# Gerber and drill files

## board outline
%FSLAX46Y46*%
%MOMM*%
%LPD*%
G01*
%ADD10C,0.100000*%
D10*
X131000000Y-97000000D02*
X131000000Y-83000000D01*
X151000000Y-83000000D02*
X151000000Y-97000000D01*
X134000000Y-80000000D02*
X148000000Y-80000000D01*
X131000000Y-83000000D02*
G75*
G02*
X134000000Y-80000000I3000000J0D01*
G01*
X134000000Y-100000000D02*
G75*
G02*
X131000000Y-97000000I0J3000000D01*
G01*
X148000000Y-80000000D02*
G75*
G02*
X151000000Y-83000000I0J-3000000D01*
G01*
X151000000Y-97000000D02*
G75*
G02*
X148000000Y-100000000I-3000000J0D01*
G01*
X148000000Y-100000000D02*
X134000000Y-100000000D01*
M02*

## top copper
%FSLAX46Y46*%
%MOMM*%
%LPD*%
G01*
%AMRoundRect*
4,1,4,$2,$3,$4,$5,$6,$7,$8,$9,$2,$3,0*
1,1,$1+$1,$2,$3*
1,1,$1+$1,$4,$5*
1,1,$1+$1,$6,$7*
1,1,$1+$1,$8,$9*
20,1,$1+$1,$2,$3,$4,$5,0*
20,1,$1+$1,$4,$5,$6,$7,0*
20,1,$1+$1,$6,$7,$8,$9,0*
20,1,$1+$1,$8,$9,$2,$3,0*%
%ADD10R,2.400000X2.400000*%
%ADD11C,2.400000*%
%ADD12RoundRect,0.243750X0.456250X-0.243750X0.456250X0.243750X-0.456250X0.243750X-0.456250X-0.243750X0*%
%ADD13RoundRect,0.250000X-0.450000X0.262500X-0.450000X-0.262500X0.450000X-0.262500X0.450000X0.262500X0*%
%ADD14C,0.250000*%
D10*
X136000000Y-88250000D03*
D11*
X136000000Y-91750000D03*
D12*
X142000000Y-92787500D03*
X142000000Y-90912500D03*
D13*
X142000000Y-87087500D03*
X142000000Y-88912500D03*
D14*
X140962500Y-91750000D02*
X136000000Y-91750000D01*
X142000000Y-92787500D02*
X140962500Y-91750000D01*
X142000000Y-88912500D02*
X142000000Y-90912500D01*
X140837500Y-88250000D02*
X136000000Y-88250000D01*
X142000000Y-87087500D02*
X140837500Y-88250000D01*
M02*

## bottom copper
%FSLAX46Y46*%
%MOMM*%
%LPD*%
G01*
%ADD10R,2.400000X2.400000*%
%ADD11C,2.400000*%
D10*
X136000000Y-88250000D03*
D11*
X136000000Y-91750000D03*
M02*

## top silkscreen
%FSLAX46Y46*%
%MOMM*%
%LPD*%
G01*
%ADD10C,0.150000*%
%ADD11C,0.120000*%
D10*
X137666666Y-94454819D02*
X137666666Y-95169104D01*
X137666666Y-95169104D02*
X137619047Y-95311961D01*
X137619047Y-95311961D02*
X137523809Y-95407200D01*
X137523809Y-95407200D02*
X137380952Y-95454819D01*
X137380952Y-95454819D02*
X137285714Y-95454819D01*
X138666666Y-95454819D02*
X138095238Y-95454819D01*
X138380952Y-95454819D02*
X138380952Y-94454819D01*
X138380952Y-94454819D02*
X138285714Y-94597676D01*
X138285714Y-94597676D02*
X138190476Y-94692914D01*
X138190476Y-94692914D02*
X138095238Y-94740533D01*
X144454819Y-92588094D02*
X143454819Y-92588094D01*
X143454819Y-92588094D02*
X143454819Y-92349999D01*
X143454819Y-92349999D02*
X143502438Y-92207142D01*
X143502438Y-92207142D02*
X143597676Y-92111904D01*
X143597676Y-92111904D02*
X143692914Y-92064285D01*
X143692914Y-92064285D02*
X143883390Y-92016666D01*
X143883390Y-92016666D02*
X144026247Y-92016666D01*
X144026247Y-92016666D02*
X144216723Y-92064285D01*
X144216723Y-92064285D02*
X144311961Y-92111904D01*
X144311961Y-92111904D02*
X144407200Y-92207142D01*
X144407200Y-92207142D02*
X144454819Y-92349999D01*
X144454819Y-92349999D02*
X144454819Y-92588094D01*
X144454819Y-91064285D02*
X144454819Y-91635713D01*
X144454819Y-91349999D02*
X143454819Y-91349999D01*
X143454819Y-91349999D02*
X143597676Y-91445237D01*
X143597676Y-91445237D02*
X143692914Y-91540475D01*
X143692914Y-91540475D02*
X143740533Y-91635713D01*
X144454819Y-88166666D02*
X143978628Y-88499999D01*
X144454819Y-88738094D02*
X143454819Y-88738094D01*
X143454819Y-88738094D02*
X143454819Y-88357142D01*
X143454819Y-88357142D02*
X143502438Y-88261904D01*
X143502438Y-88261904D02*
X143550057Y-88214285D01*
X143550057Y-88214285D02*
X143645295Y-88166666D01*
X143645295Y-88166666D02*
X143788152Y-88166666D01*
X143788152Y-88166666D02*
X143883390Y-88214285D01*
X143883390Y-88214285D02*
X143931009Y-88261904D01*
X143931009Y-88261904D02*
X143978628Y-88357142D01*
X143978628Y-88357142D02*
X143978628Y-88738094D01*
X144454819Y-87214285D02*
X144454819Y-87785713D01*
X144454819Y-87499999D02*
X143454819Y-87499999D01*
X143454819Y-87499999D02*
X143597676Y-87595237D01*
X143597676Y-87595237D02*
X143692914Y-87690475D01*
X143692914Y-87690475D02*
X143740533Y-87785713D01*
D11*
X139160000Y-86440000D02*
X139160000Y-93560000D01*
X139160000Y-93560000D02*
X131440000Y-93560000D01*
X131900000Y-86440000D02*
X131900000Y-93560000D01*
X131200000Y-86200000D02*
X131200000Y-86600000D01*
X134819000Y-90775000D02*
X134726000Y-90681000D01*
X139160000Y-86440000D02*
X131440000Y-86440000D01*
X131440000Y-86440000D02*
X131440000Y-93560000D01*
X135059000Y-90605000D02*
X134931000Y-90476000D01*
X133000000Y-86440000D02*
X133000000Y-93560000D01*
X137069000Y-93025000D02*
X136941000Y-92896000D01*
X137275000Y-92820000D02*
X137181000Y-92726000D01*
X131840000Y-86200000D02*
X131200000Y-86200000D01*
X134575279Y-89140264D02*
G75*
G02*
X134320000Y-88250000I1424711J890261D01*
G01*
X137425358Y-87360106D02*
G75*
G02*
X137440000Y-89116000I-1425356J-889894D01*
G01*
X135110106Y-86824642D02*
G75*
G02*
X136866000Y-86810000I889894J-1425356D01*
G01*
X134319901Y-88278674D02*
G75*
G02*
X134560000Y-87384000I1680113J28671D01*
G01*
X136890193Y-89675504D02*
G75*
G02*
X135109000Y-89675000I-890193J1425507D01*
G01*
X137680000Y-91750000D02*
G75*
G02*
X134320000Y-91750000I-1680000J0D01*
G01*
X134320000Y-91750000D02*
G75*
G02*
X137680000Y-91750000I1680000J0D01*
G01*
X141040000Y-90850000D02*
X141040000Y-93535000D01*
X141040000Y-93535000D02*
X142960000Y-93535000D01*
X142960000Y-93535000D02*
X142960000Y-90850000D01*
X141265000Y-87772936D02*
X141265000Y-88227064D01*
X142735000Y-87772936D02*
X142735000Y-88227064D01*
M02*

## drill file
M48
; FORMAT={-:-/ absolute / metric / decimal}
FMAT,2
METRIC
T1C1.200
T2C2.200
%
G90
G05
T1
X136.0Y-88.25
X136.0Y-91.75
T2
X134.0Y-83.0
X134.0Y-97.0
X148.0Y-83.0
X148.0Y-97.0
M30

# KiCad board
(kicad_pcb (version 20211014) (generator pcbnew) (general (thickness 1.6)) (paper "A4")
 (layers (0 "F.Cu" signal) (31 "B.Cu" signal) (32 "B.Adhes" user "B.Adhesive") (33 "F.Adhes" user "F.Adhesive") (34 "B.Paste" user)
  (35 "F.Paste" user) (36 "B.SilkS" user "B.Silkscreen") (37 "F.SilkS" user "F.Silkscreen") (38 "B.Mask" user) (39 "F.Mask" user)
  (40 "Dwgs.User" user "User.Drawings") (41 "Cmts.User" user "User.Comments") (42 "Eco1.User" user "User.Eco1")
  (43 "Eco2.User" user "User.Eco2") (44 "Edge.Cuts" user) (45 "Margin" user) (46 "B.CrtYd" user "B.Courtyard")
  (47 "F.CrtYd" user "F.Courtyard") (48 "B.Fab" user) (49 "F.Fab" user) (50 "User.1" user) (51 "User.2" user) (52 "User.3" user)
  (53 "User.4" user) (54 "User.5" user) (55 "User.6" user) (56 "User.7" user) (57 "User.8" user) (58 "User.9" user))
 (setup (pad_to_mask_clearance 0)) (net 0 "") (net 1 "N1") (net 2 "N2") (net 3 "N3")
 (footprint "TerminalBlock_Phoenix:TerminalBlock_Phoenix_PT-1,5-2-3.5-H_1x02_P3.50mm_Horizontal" (layer "F.Cu") (at 136 88.25 -90)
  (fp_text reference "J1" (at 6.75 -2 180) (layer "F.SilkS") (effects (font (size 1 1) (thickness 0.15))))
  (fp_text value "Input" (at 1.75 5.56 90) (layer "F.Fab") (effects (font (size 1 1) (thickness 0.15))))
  (fp_line (start -1.81 -3.16) (end 5.31 -3.16) (layer "F.SilkS") (width 0.12))
  (fp_line (start 5.31 -3.16) (end 5.31 4.56) (layer "F.SilkS") (width 0.12))
  (fp_line (start -1.81 4.1) (end 5.31 4.1) (layer "F.SilkS") (width 0.12))
  (fp_line (start -2.05 4.8) (end -1.65 4.8) (layer "F.SilkS") (width 0.12))
  (fp_line (start 2.525 1.181) (end 2.431 1.274) (layer "F.SilkS") (width 0.12))
  (fp_line (start -1.81 -3.16) (end -1.81 4.56) (layer "F.SilkS") (width 0.12))
  (fp_line (start -1.81 4.56) (end 5.31 4.56) (layer "F.SilkS") (width 0.12))
  (fp_line (start 2.355 0.941) (end 2.226 1.069) (layer "F.SilkS") (width 0.12))
  (fp_line (start -1.81 3) (end 5.31 3) (layer "F.SilkS") (width 0.12))
  (fp_line (start 4.775 -1.069) (end 4.646 -0.941) (layer "F.SilkS") (width 0.12))
  (fp_line (start 4.57 -1.275) (end 4.476 -1.181) (layer "F.SilkS") (width 0.12))
  (fp_line (start -2.05 4.16) (end -2.05 4.8) (layer "F.SilkS") (width 0.12))
  (fp_arc (start 0.890264 1.424721) (mid 0.463071 1.61492) (end 0 1.68) (layer "F.SilkS") (width 0.12))
  (fp_arc (start -0.889894 -1.425358) (mid -0.014012 -1.680286) (end 0.866 -1.44) (layer "F.SilkS") (width 0.12))
  (fp_arc (start -1.425358 0.889894) (mid -1.680286 0.014012) (end -1.44 -0.866) (layer "F.SilkS") (width 0.12))
  (fp_arc (start 0.028674 1.680099) (mid -0.435535 1.622918) (end -0.866 1.44) (layer "F.SilkS") (width 0.12))
  (fp_arc (start 1.425504 -0.890193) (mid 1.680626 0.000476) (end 1.425 0.891) (layer "F.SilkS") (width 0.12))
  (fp_circle (center 3.5 0) (end 5.18 0) (layer "F.SilkS") (width 0.12) (fill none))
  (pad "1" thru_hole rect (at 0 0 270) (size 2.4 2.4) (drill 1.2) (layers *.Cu *.Mask) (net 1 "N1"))
  (pad "2" thru_hole circle (at 3.5 0 270) (size 2.4 2.4) (drill 1.2) (layers *.Cu *.Mask) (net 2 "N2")))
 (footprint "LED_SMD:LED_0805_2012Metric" (layer "F.Cu") (at 142 91.85 90)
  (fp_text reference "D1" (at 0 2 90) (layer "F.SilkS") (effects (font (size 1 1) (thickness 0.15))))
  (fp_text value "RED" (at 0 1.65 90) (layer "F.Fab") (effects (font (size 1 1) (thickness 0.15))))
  (fp_line (start 1 -0.96) (end -1.685 -0.96) (layer "F.SilkS") (width 0.12))
  (fp_line (start -1.685 -0.96) (end -1.685 0.96) (layer "F.SilkS") (width 0.12))
  (fp_line (start -1.685 0.96) (end 1 0.96) (layer "F.SilkS") (width 0.12))
  (pad "1" smd roundrect (at -0.9375 0 90) (size 0.975 1.4) (layers "F.Cu" "F.Paste" "F.Mask") (roundrect_rratio 0.25) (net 2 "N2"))
  (pad "2" smd roundrect (at 0.9375 0 90) (size 0.975 1.4) (layers "F.Cu" "F.Paste" "F.Mask") (roundrect_rratio 0.25) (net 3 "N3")))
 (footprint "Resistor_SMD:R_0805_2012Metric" (layer "F.Cu") (at 142 88 -90)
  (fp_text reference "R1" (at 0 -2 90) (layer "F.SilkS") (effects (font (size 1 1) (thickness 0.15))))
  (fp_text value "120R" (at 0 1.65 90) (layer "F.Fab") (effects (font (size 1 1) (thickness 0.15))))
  (fp_line (start -0.227064 0.735) (end 0.227064 0.735) (layer "F.SilkS") (width 0.12))
  (fp_line (start -0.227064 -0.735) (end 0.227064 -0.735) (layer "F.SilkS") (width 0.12))
  (pad "1" smd roundrect (at -0.9125 0 270) (size 1.025 1.4) (layers "F.Cu" "F.Paste" "F.Mask") (roundrect_rratio 0.243902) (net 1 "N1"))
  (pad "2" smd roundrect (at 0.9125 0 270) (size 1.025 1.4) (layers "F.Cu" "F.Paste" "F.Mask") (roundrect_rratio 0.243902) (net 3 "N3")))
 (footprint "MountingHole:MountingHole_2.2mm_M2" (layer "F.Cu") (at 148 83)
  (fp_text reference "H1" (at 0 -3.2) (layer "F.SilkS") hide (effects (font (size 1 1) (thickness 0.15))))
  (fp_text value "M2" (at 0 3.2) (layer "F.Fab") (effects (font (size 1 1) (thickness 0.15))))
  (pad "" np_thru_hole circle (at 0 0) (size 2.2 2.2) (drill 2.2) (layers *.Cu *.Mask)))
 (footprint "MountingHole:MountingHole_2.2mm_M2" (layer "F.Cu") (at 148 97)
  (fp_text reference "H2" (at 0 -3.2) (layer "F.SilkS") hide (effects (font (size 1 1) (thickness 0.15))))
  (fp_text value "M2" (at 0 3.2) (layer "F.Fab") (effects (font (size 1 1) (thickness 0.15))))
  (pad "" np_thru_hole circle (at 0 0) (size 2.2 2.2) (drill 2.2) (layers *.Cu *.Mask)))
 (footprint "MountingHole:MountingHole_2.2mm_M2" (layer "F.Cu") (at 134 83)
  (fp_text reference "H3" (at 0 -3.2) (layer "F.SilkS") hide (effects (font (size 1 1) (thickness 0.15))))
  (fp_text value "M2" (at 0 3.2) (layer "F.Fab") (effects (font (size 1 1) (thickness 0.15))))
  (pad "" np_thru_hole circle (at 0 0) (size 2.2 2.2) (drill 2.2) (layers *.Cu *.Mask)))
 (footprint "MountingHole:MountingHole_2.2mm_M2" (layer "F.Cu") (at 134 97)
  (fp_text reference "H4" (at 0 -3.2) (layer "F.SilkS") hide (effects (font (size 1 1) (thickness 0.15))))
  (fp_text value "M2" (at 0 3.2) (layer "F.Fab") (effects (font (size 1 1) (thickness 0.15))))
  (pad "" np_thru_hole circle (at 0 0) (size 2.2 2.2) (drill 2.2) (layers *.Cu *.Mask)))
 (gr_line (start 131 97) (end 131 83) (layer "Edge.Cuts") (width 0.1))
 (gr_line (start 151 83) (end 151 97) (layer "Edge.Cuts") (width 0.1))
 (gr_line (start 134 80) (end 148 80) (layer "Edge.Cuts") (width 0.1))
 (gr_arc (start 131 83) (mid 131.87868 80.87868) (end 134 80) (layer "Edge.Cuts") (width 0.1))
 (gr_arc (start 134 100) (mid 131.87868 99.12132) (end 131 97) (layer "Edge.Cuts") (width 0.1))
 (gr_arc (start 148 80) (mid 150.12132 80.87868) (end 151 83) (layer "Edge.Cuts") (width 0.1))
 (gr_arc (start 151 97) (mid 150.12132 99.12132) (end 148 100) (layer "Edge.Cuts") (width 0.1))
 (gr_line (start 148 100) (end 134 100) (layer "Edge.Cuts") (width 0.1))
 (segment (start 140.9625 91.75) (end 136 91.75) (width 0.25) (layer "F.Cu") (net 2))
 (segment (start 142 92.7875) (end 140.9625 91.75) (width 0.25) (layer "F.Cu") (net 2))
 (segment (start 142 88.9125) (end 142 90.9125) (width 0.25) (layer "F.Cu") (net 3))
 (segment (start 140.8375 88.25) (end 136 88.25) (width 0.25) (layer "F.Cu") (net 1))
 (segment (start 142 87.0875) (end 140.8375 88.25) (width 0.25) (layer "F.Cu") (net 1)))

